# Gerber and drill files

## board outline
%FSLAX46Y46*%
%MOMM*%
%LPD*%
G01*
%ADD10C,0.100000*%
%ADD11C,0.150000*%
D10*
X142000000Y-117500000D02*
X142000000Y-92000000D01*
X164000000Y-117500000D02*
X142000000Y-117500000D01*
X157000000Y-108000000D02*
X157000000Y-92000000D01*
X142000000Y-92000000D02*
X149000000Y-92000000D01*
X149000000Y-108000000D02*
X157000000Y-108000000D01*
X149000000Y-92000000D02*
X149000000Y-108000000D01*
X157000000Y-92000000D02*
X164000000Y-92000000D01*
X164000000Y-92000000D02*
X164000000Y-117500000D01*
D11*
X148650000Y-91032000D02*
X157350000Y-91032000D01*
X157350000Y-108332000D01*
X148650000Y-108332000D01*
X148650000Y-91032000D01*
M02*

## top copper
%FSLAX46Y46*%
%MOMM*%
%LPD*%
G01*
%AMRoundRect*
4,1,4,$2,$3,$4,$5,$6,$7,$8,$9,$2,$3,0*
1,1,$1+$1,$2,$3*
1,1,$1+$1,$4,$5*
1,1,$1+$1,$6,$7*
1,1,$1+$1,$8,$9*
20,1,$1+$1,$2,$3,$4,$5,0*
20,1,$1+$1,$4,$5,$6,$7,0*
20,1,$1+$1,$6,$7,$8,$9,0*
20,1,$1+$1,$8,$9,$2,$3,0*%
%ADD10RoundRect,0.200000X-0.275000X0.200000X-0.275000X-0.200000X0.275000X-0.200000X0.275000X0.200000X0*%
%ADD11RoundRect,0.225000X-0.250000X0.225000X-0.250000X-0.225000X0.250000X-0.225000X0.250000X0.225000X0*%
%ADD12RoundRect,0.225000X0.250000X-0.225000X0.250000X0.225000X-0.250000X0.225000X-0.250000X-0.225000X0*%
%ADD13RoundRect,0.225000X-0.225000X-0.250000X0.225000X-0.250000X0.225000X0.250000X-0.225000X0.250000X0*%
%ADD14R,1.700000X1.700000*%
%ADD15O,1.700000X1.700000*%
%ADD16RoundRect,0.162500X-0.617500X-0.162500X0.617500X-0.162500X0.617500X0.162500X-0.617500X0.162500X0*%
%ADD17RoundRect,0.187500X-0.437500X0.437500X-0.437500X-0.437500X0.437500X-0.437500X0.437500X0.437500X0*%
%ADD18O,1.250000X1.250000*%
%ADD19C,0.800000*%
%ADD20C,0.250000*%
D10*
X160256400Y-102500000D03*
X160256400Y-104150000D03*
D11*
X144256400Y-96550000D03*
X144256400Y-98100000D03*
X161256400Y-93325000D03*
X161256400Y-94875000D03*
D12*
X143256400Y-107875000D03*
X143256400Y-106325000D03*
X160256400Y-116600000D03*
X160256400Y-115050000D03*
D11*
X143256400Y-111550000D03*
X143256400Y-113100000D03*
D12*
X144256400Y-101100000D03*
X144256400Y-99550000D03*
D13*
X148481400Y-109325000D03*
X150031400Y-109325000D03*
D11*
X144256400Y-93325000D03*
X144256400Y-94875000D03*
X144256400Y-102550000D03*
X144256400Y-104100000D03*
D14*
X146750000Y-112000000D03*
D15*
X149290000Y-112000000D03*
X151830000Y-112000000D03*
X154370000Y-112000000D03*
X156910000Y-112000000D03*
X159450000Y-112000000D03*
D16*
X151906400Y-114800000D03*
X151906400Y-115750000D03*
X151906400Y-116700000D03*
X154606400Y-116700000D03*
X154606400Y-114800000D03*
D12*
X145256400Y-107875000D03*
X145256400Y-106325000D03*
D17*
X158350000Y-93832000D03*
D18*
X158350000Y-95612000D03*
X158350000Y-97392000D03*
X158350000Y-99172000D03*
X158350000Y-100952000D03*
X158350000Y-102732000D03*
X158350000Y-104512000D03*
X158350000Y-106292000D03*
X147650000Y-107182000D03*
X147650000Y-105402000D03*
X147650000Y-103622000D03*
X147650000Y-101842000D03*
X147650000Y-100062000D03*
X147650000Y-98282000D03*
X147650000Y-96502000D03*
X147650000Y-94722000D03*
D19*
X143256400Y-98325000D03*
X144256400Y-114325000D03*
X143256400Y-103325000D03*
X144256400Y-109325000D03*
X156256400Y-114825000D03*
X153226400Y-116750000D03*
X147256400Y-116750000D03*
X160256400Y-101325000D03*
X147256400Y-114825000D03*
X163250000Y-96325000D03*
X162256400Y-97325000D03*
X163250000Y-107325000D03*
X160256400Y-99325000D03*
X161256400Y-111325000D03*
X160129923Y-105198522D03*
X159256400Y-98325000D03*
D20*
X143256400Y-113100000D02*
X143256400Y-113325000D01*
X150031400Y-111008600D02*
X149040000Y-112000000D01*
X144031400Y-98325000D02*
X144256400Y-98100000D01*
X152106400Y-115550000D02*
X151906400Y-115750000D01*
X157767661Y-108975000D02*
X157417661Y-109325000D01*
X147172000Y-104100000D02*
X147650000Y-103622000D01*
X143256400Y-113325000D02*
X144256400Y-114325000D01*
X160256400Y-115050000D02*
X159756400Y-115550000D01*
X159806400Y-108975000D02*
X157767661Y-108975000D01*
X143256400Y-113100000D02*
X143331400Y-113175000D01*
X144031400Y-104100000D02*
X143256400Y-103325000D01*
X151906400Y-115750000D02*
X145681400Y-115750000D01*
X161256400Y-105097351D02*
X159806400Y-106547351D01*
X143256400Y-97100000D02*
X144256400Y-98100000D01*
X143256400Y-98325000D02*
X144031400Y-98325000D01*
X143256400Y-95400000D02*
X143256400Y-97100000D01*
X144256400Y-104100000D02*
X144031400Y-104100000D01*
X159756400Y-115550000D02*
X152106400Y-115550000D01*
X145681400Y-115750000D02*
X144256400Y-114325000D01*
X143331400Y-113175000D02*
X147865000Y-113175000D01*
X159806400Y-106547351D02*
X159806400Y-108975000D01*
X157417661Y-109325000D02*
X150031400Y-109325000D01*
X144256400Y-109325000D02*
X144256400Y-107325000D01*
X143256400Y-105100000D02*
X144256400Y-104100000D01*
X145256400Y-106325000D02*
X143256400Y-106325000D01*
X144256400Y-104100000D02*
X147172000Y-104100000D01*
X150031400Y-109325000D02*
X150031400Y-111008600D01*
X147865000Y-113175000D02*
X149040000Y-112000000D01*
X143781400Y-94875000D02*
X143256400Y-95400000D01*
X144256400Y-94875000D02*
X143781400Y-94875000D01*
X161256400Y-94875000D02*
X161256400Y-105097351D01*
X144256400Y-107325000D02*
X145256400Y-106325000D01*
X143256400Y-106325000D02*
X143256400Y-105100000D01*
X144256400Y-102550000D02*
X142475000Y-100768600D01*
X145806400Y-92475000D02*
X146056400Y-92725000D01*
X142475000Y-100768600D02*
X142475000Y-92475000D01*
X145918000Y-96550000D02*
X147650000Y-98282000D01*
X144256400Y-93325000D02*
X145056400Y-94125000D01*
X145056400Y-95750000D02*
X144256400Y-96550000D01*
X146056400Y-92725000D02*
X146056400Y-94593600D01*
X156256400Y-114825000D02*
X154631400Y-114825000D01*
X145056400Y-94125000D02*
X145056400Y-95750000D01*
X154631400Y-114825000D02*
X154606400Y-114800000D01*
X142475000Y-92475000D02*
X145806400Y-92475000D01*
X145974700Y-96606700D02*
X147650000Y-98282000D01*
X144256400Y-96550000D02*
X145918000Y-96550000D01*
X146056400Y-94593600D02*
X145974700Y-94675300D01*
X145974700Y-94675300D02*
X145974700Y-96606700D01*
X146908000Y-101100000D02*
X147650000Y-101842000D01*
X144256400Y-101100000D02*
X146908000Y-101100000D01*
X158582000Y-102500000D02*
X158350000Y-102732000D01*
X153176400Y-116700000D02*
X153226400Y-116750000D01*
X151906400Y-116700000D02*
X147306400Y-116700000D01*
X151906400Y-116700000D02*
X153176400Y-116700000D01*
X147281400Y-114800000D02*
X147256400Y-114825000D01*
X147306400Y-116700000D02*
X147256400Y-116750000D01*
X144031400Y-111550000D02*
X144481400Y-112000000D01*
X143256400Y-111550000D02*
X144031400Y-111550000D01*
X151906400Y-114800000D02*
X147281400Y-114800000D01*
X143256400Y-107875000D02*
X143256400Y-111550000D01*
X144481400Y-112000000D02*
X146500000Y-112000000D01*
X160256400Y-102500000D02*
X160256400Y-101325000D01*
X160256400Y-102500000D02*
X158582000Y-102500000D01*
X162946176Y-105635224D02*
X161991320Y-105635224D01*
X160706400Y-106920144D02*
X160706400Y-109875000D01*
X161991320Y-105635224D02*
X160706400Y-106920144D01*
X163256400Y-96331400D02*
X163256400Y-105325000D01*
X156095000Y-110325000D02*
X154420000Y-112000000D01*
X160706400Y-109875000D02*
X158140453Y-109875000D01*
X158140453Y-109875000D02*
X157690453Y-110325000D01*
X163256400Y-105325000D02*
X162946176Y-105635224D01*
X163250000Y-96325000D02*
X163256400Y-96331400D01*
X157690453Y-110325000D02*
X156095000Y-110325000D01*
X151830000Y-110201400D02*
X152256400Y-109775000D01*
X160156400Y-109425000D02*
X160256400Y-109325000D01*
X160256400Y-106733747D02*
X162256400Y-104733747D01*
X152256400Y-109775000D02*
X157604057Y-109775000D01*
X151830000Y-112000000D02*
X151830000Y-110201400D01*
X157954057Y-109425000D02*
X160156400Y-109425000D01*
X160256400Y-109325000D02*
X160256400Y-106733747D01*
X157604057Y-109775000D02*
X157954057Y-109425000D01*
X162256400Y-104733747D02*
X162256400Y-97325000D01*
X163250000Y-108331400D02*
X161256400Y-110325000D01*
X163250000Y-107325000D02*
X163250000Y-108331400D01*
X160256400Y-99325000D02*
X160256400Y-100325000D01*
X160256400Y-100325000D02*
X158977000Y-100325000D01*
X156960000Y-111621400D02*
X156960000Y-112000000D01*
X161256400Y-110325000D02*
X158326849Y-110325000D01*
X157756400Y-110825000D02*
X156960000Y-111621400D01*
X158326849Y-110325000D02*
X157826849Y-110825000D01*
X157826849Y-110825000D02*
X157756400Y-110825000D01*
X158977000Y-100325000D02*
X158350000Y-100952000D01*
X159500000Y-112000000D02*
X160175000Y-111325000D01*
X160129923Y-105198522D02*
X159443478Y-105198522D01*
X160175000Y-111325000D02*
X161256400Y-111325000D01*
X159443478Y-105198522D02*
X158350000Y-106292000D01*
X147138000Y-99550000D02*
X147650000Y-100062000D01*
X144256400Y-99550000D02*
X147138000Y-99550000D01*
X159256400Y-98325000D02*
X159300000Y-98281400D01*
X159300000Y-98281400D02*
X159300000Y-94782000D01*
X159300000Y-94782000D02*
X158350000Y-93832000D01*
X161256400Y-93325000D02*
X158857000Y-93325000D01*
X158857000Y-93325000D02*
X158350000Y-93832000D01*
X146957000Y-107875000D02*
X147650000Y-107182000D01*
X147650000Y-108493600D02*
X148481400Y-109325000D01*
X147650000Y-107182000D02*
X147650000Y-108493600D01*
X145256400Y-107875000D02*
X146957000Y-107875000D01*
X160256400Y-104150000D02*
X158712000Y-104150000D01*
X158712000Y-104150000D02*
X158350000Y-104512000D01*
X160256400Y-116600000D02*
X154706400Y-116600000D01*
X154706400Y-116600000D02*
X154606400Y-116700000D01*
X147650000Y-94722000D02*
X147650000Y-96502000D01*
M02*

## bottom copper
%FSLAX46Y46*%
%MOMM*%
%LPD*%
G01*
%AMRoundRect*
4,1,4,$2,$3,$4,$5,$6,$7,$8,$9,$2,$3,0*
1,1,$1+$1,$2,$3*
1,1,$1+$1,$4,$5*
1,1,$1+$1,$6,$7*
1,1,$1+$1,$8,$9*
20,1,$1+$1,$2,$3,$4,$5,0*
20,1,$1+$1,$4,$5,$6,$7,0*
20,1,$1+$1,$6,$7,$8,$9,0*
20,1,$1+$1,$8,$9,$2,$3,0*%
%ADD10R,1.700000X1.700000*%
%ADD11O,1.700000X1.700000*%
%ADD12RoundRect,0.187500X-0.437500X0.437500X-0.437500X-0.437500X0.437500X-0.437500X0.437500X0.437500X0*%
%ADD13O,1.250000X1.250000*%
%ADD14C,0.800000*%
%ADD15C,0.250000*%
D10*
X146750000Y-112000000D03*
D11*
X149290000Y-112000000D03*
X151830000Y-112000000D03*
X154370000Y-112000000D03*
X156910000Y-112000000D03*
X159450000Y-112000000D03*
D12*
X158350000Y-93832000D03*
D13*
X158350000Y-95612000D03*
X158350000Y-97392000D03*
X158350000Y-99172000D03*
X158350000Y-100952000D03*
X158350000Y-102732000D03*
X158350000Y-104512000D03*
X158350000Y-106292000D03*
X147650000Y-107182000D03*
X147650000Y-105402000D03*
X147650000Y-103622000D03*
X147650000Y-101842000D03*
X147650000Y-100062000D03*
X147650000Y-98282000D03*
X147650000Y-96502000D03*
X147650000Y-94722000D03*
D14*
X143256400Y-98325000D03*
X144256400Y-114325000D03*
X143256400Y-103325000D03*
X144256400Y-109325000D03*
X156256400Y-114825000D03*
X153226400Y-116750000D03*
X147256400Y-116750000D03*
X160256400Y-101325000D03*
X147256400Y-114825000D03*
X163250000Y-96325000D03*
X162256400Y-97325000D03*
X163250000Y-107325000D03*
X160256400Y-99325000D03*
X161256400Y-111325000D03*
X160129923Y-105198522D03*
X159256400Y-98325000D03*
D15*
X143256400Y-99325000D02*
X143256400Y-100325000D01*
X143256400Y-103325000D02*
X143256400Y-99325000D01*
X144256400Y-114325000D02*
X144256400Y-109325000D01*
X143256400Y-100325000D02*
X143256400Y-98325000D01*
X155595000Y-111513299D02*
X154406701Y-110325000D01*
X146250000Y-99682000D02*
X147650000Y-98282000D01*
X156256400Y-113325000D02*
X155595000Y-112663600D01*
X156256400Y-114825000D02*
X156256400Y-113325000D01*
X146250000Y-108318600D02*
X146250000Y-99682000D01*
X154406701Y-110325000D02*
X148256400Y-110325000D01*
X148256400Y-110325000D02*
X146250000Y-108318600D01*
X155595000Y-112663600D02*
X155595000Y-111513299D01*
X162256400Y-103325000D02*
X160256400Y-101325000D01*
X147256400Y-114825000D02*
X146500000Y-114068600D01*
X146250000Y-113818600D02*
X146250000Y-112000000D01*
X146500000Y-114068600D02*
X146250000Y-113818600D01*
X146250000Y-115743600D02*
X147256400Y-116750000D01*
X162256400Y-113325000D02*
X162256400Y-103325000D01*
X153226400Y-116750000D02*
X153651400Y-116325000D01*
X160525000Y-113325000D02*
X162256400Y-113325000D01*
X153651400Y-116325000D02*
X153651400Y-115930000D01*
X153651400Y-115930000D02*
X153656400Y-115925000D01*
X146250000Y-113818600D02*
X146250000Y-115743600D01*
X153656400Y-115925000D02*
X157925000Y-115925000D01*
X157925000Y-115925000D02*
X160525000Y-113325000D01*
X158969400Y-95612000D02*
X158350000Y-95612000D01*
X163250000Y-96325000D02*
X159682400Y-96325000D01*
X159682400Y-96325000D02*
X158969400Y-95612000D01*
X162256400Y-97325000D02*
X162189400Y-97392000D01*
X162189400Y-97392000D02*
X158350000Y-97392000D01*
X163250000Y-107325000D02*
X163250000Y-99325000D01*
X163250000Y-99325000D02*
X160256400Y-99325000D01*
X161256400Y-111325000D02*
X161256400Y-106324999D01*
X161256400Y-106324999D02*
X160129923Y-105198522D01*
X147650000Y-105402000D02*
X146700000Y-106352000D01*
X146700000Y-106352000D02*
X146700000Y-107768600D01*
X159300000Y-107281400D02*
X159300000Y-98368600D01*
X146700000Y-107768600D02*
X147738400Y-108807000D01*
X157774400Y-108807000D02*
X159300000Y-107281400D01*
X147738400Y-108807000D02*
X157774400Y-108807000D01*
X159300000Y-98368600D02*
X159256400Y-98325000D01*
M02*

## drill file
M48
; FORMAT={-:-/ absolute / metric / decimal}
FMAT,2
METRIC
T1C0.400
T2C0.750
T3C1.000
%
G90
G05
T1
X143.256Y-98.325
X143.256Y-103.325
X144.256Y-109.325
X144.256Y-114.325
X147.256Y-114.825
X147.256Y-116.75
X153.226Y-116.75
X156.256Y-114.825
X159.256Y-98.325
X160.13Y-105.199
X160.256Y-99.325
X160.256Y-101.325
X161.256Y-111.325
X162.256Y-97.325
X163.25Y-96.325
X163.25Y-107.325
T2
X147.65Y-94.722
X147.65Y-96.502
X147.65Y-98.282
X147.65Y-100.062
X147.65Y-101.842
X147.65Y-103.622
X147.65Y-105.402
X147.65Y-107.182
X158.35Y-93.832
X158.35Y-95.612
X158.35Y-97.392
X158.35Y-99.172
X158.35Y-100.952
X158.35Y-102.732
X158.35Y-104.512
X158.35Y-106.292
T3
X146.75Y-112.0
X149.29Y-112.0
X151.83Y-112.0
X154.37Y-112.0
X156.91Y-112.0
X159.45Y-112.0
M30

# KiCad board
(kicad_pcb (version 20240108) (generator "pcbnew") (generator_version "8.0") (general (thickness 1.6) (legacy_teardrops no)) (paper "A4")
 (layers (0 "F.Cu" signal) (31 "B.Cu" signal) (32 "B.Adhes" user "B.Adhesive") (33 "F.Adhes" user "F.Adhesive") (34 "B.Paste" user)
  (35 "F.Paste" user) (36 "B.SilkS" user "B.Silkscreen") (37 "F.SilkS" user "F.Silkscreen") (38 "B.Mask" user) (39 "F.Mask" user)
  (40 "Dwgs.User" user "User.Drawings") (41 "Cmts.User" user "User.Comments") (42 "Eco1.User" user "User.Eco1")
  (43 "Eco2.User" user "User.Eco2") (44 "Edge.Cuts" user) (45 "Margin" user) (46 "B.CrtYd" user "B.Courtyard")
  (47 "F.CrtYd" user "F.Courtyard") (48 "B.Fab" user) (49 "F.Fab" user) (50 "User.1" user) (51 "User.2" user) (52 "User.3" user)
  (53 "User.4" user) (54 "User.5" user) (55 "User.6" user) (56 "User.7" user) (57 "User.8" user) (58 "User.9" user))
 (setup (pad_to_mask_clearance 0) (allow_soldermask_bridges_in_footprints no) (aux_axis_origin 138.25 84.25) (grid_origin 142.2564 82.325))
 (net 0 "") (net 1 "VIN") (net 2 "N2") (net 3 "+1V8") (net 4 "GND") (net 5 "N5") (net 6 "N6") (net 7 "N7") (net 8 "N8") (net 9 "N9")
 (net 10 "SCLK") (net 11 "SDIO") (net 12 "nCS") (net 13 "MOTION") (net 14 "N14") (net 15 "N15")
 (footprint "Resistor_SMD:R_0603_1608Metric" (layer "F.Cu") (at 160.2564 103.325 -90)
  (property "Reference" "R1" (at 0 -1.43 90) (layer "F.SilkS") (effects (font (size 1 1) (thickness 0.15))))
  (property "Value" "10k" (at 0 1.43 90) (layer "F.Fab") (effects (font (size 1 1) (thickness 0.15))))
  (pad "1" smd roundrect (at -0.825 0 270) (size 0.8 0.95) (layers "F.Cu" "F.Paste" "F.Mask") (roundrect_rratio 0.25) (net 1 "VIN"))
  (pad "2" smd roundrect (at 0.825 0 270) (size 0.8 0.95) (layers "F.Cu" "F.Paste" "F.Mask") (roundrect_rratio 0.25) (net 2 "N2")))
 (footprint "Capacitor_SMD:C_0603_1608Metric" (layer "F.Cu") (at 144.2564 97.325 -90)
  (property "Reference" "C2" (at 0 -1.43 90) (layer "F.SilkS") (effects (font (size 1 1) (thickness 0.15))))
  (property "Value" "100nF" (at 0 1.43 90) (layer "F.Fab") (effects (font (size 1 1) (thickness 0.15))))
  (pad "1" smd roundrect (at -0.775 0 270) (size 0.9 0.95) (layers "F.Cu" "F.Paste" "F.Mask") (roundrect_rratio 0.25) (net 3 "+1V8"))
  (pad "2" smd roundrect (at 0.775 0 270) (size 0.9 0.95) (layers "F.Cu" "F.Paste" "F.Mask") (roundrect_rratio 0.25) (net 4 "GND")))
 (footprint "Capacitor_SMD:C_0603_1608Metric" (layer "F.Cu") (at 161.2564 94.1 -90)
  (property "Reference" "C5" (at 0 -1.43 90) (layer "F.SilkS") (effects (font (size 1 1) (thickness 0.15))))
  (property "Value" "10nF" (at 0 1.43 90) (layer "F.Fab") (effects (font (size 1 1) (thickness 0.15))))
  (pad "1" smd roundrect (at -0.775 0 270) (size 0.9 0.95) (layers "F.Cu" "F.Paste" "F.Mask") (roundrect_rratio 0.25) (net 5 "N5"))
  (pad "2" smd roundrect (at 0.775 0 270) (size 0.9 0.95) (layers "F.Cu" "F.Paste" "F.Mask") (roundrect_rratio 0.25) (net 4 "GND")))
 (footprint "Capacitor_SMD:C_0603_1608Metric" (layer "F.Cu") (at 143.2564 107.1 90)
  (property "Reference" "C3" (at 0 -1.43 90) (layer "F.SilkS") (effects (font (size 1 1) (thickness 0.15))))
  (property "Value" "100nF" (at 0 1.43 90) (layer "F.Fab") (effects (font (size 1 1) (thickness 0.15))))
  (pad "1" smd roundrect (at -0.775 0 90) (size 0.9 0.95) (layers "F.Cu" "F.Paste" "F.Mask") (roundrect_rratio 0.25) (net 1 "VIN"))
  (pad "2" smd roundrect (at 0.775 0 90) (size 0.9 0.95) (layers "F.Cu" "F.Paste" "F.Mask") (roundrect_rratio 0.25) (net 4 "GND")))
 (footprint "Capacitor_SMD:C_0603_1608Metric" (layer "F.Cu") (at 160.2564 115.825 90)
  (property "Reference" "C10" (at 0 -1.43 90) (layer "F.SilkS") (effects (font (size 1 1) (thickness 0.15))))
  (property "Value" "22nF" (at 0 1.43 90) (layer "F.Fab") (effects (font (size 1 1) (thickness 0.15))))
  (pad "1" smd roundrect (at -0.775 0 90) (size 0.9 0.95) (layers "F.Cu" "F.Paste" "F.Mask") (roundrect_rratio 0.25) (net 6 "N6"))
  (pad "2" smd roundrect (at 0.775 0 90) (size 0.9 0.95) (layers "F.Cu" "F.Paste" "F.Mask") (roundrect_rratio 0.25) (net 4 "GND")))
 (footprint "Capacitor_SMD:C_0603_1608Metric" (layer "F.Cu") (at 143.2564 112.325 -90)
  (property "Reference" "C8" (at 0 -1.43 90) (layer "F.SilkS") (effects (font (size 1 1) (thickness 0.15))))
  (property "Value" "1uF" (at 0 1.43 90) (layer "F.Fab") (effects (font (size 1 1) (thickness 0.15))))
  (pad "1" smd roundrect (at -0.775 0 270) (size 0.9 0.95) (layers "F.Cu" "F.Paste" "F.Mask") (roundrect_rratio 0.25) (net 1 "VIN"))
  (pad "2" smd roundrect (at 0.775 0 270) (size 0.9 0.95) (layers "F.Cu" "F.Paste" "F.Mask") (roundrect_rratio 0.25) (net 4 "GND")))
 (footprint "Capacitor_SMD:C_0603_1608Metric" (layer "F.Cu") (at 144.2564 100.325 90)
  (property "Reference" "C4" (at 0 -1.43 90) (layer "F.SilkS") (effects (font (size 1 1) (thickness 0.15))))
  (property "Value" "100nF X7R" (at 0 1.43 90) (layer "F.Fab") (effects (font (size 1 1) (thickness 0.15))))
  (pad "1" smd roundrect (at -0.775 0 90) (size 0.9 0.95) (layers "F.Cu" "F.Paste" "F.Mask") (roundrect_rratio 0.25) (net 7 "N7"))
  (pad "2" smd roundrect (at 0.775 0 90) (size 0.9 0.95) (layers "F.Cu" "F.Paste" "F.Mask") (roundrect_rratio 0.25) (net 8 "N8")))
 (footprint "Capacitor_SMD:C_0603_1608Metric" (layer "F.Cu") (at 149.2564 109.325)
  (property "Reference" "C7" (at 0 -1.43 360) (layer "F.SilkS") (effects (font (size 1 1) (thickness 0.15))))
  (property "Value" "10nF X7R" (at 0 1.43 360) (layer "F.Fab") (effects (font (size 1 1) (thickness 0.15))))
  (pad "1" smd roundrect (at -0.775 0) (size 0.9 0.95) (layers "F.Cu" "F.Paste" "F.Mask") (roundrect_rratio 0.25) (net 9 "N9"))
  (pad "2" smd roundrect (at 0.775 0) (size 0.9 0.95) (layers "F.Cu" "F.Paste" "F.Mask") (roundrect_rratio 0.25) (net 4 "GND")))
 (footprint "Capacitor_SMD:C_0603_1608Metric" (layer "F.Cu") (at 144.2564 94.1 -90)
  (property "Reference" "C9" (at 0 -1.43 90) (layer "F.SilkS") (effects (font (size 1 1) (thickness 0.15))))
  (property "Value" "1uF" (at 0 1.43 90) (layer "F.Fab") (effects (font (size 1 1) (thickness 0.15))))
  (pad "1" smd roundrect (at -0.775 0 270) (size 0.9 0.95) (layers "F.Cu" "F.Paste" "F.Mask") (roundrect_rratio 0.25) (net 3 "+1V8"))
  (pad "2" smd roundrect (at 0.775 0 270) (size 0.9 0.95) (layers "F.Cu" "F.Paste" "F.Mask") (roundrect_rratio 0.25) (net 4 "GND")))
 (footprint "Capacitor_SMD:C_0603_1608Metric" (layer "F.Cu") (at 144.2564 103.325 -90)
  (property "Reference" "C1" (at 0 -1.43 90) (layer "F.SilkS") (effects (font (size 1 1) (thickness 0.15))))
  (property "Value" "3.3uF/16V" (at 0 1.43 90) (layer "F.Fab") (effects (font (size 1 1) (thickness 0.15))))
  (pad "1" smd roundrect (at -0.775 0 270) (size 0.9 0.95) (layers "F.Cu" "F.Paste" "F.Mask") (roundrect_rratio 0.25) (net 3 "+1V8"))
  (pad "2" smd roundrect (at 0.775 0 270) (size 0.9 0.95) (layers "F.Cu" "F.Paste" "F.Mask") (roundrect_rratio 0.25) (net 4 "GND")))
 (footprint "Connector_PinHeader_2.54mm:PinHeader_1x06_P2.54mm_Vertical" (layer "F.Cu") (at 146.75 112 90)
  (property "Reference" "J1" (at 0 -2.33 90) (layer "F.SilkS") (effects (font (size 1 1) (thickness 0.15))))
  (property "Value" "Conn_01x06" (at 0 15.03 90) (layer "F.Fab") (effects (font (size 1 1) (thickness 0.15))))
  (pad "1" thru_hole rect (at 0 0 90) (size 1.7 1.7) (drill 1) (layers "*.Cu" "*.Mask") (remove_unused_layers no) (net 1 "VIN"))
  (pad "2" thru_hole oval (at 0 2.54 90) (size 1.7 1.7) (drill 1) (layers "*.Cu" "*.Mask") (remove_unused_layers no) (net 4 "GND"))
  (pad "3" thru_hole oval (at 0 5.08 90) (size 1.7 1.7) (drill 1) (layers "*.Cu" "*.Mask") (remove_unused_layers no) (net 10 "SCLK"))
  (pad "4" thru_hole oval (at 0 7.62 90) (size 1.7 1.7) (drill 1) (layers "*.Cu" "*.Mask") (remove_unused_layers no) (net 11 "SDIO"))
  (pad "5" thru_hole oval (at 0 10.16 90) (size 1.7 1.7) (drill 1) (layers "*.Cu" "*.Mask") (remove_unused_layers no) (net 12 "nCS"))
  (pad "6" thru_hole oval (at 0 12.7 90) (size 1.7 1.7) (drill 1) (layers "*.Cu" "*.Mask") (remove_unused_layers no) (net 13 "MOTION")))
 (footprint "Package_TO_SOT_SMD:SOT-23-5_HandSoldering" (layer "F.Cu") (at 153.2564 115.75)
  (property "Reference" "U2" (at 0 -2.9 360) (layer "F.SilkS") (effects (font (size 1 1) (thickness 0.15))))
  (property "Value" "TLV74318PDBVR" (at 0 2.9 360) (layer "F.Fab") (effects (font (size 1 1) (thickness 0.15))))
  (pad "1" smd roundrect (at -1.35 -0.95) (size 1.56 0.65) (layers "F.Cu" "F.Paste" "F.Mask") (roundrect_rratio 0.25) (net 1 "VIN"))
  (pad "2" smd roundrect (at -1.35 0) (size 1.56 0.65) (layers "F.Cu" "F.Paste" "F.Mask") (roundrect_rratio 0.25) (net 4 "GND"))
  (pad "3" smd roundrect (at -1.35 0.95) (size 1.56 0.65) (layers "F.Cu" "F.Paste" "F.Mask") (roundrect_rratio 0.25) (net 1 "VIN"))
  (pad "4" smd roundrect (at 1.35 0.95) (size 1.56 0.65) (layers "F.Cu" "F.Paste" "F.Mask") (roundrect_rratio 0.25) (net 6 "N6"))
  (pad "5" smd roundrect (at 1.35 -0.95) (size 1.56 0.65) (layers "F.Cu" "F.Paste" "F.Mask") (roundrect_rratio 0.25) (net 3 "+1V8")))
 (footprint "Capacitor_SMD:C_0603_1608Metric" (layer "F.Cu") (at 145.2564 107.1 90)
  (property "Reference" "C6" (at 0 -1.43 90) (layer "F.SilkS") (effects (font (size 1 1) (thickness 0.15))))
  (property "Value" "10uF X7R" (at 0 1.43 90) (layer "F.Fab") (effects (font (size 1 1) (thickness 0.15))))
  (pad "1" smd roundrect (at -0.775 0 90) (size 0.9 0.95) (layers "F.Cu" "F.Paste" "F.Mask") (roundrect_rratio 0.25) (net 9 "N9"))
  (pad "2" smd roundrect (at 0.775 0 90) (size 0.9 0.95) (layers "F.Cu" "F.Paste" "F.Mask") (roundrect_rratio 0.25) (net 4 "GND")))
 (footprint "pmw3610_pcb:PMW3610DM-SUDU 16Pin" (layer "B.Cu") (at 153 100 90)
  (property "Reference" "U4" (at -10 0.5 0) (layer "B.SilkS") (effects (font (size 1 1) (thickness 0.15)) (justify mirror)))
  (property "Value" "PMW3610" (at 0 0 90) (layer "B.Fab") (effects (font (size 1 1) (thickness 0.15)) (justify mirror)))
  (fp_rect (start -8.332 -4.35) (end 8.968 4.35) (stroke (width 0.15) (type solid)) (fill none) (layer "Edge.Cuts"))
  (pad "1" thru_hole roundrect (at 6.168 5.35 270) (size 1.25 1.25) (drill 0.75) (layers "*.Cu" "*.Mask") (remove_unused_layers no)
   (roundrect_rratio 0.15) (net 5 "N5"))
  (pad "2" thru_hole oval (at 4.388 5.35 270) (size 1.25 1.25) (drill 0.75) (layers "*.Cu" "*.Mask") (remove_unused_layers no)
   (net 11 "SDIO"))
  (pad "3" thru_hole oval (at 2.608 5.35 270) (size 1.25 1.25) (drill 0.75) (layers "*.Cu" "*.Mask") (remove_unused_layers no)
   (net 10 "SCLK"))
  (pad "4" thru_hole oval (at 0.828 5.35 270) (size 1.25 1.25) (drill 0.75) (layers "*.Cu" "*.Mask") (remove_unused_layers no)
   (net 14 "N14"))
  (pad "5" thru_hole oval (at -0.952 5.35 270) (size 1.25 1.25) (drill 0.75) (layers "*.Cu" "*.Mask") (remove_unused_layers no)
   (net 12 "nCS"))
  (pad "6" thru_hole oval (at -2.732 5.35 270) (size 1.25 1.25) (drill 0.75) (layers "*.Cu" "*.Mask") (remove_unused_layers no)
   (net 1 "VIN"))
  (pad "7" thru_hole oval (at -4.512 5.35 270) (size 1.25 1.25) (drill 0.75) (layers "*.Cu" "*.Mask") (remove_unused_layers no) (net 2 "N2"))
  (pad "8" thru_hole oval (at -6.292 5.35 270) (size 1.25 1.25) (drill 0.75) (layers "*.Cu" "*.Mask") (remove_unused_layers no)
   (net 13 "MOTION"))
  (pad "9" thru_hole oval (at -7.182 -5.35 270) (size 1.25 1.25) (drill 0.75) (layers "*.Cu" "*.Mask") (remove_unused_layers no)
   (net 9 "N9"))
  (pad "10" thru_hole oval (at -5.402 -5.35 270) (size 1.25 1.25) (drill 0.75) (layers "*.Cu" "*.Mask") (remove_unused_layers no)
   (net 5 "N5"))
  (pad "11" thru_hole oval (at -3.622 -5.35 270) (size 1.25 1.25) (drill 0.75) (layers "*.Cu" "*.Mask") (remove_unused_layers no)
   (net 4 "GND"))
  (pad "12" thru_hole oval (at -1.842 -5.35 270) (size 1.25 1.25) (drill 0.75) (layers "*.Cu" "*.Mask") (remove_unused_layers no)
   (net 7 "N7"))
  (pad "13" thru_hole oval (at -0.062 -5.35 270) (size 1.25 1.25) (drill 0.75) (layers "*.Cu" "*.Mask") (remove_unused_layers no)
   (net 8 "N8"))
  (pad "14" thru_hole oval (at 1.718 -5.35 270) (size 1.25 1.25) (drill 0.75) (layers "*.Cu" "*.Mask") (remove_unused_layers no)
   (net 3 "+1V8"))
  (pad "15" thru_hole oval (at 3.498 -5.35 270) (size 1.25 1.25) (drill 0.75) (layers "*.Cu" "*.Mask") (remove_unused_layers no)
   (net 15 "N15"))
  (pad "16" thru_hole oval (at 5.278 -5.35 270) (size 1.25 1.25) (drill 0.75) (layers "*.Cu" "*.Mask") (remove_unused_layers no)
   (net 15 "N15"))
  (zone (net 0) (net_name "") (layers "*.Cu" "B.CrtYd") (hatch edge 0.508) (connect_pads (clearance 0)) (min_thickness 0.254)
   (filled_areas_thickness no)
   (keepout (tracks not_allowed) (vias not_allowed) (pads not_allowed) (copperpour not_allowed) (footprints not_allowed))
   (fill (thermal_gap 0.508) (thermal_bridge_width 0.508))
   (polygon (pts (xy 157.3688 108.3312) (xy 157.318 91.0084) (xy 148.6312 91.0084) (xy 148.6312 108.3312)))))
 (gr_line (start 142 117.5) (end 142 92) (stroke (width 0.1) (type default)) (layer "Edge.Cuts"))
 (gr_line (start 164 117.5) (end 142 117.5) (stroke (width 0.1) (type default)) (layer "Edge.Cuts"))
 (gr_line (start 157 108) (end 157 92) (stroke (width 0.1) (type default)) (layer "Edge.Cuts"))
 (gr_line (start 142 92) (end 149 92) (stroke (width 0.1) (type default)) (layer "Edge.Cuts"))
 (gr_line (start 149 108) (end 157 108) (stroke (width 0.1) (type default)) (layer "Edge.Cuts"))
 (gr_line (start 149 92) (end 149 108) (stroke (width 0.1) (type default)) (layer "Edge.Cuts"))
 (gr_line (start 157 92) (end 164 92) (stroke (width 0.1) (type default)) (layer "Edge.Cuts"))
 (gr_line (start 164 92) (end 164 117.5) (stroke (width 0.1) (type default)) (layer "Edge.Cuts"))
 (segment (start 143.2564 113.1) (end 143.2564 113.325) (width 0.25) (layer "F.Cu") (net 4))
 (segment (start 150.0314 111.0086) (end 149.04 112) (width 0.25) (layer "F.Cu") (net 4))
 (segment (start 144.0314 98.325) (end 144.2564 98.1) (width 0.25) (layer "F.Cu") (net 4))
 (segment (start 152.1064 115.55) (end 151.9064 115.75) (width 0.25) (layer "F.Cu") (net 4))
 (segment (start 157.767661 108.975) (end 157.417661 109.325) (width 0.25) (layer "F.Cu") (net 4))
 (segment (start 147.172 104.1) (end 147.65 103.622) (width 0.25) (layer "F.Cu") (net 4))
 (segment (start 143.2564 113.325) (end 144.2564 114.325) (width 0.25) (layer "F.Cu") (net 4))
 (segment (start 160.2564 115.05) (end 159.7564 115.55) (width 0.25) (layer "F.Cu") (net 4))
 (segment (start 159.8064 108.975) (end 157.767661 108.975) (width 0.25) (layer "F.Cu") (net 4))
 (segment (start 143.2564 113.1) (end 143.3314 113.175) (width 0.25) (layer "F.Cu") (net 4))
 (segment (start 144.0314 104.1) (end 143.2564 103.325) (width 0.25) (layer "F.Cu") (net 4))
 (segment (start 151.9064 115.75) (end 145.6814 115.75) (width 0.25) (layer "F.Cu") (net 4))
 (segment (start 161.2564 105.097351) (end 159.8064 106.547351) (width 0.25) (layer "F.Cu") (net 4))
 (segment (start 143.2564 97.1) (end 144.2564 98.1) (width 0.25) (layer "F.Cu") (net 4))
 (segment (start 143.2564 98.325) (end 144.0314 98.325) (width 0.25) (layer "F.Cu") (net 4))
 (segment (start 143.2564 95.4) (end 143.2564 97.1) (width 0.25) (layer "F.Cu") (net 4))
 (segment (start 144.2564 104.1) (end 144.0314 104.1) (width 0.25) (layer "F.Cu") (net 4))
 (segment (start 159.7564 115.55) (end 152.1064 115.55) (width 0.25) (layer "F.Cu") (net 4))
 (segment (start 145.6814 115.75) (end 144.2564 114.325) (width 0.25) (layer "F.Cu") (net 4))
 (segment (start 143.3314 113.175) (end 147.865 113.175) (width 0.25) (layer "F.Cu") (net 4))
 (segment (start 159.8064 106.547351) (end 159.8064 108.975) (width 0.25) (layer "F.Cu") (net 4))
 (segment (start 157.417661 109.325) (end 150.0314 109.325) (width 0.25) (layer "F.Cu") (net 4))
 (segment (start 144.2564 109.325) (end 144.2564 107.325) (width 0.25) (layer "F.Cu") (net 4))
 (segment (start 143.2564 105.1) (end 144.2564 104.1) (width 0.25) (layer "F.Cu") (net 4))
 (segment (start 145.2564 106.325) (end 143.2564 106.325) (width 0.25) (layer "F.Cu") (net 4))
 (segment (start 144.2564 104.1) (end 147.172 104.1) (width 0.25) (layer "F.Cu") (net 4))
 (segment (start 150.0314 109.325) (end 150.0314 111.0086) (width 0.25) (layer "F.Cu") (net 4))
 (segment (start 147.865 113.175) (end 149.04 112) (width 0.25) (layer "F.Cu") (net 4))
 (segment (start 143.7814 94.875) (end 143.2564 95.4) (width 0.25) (layer "F.Cu") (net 4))
 (segment (start 144.2564 94.875) (end 143.7814 94.875) (width 0.25) (layer "F.Cu") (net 4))
 (segment (start 161.2564 94.875) (end 161.2564 105.097351) (width 0.25) (layer "F.Cu") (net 4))
 (segment (start 144.2564 107.325) (end 145.2564 106.325) (width 0.25) (layer "F.Cu") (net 4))
 (segment (start 143.2564 106.325) (end 143.2564 105.1) (width 0.25) (layer "F.Cu") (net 4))
 (via (at 143.2564 98.325) (size 0.8) (drill 0.4) (layers "F.Cu" "B.Cu") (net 4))
 (via (at 144.2564 114.325) (size 0.8) (drill 0.4) (layers "F.Cu" "B.Cu") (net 4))
 (via (at 143.2564 103.325) (size 0.8) (drill 0.4) (layers "F.Cu" "B.Cu") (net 4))
 (via (at 144.2564 109.325) (size 0.8) (drill 0.4) (layers "F.Cu" "B.Cu") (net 4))
 (segment (start 143.2564 99.325) (end 143.2564 100.325) (width 0.25) (layer "B.Cu") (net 4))
 (segment (start 143.2564 103.325) (end 143.2564 99.325) (width 0.25) (layer "B.Cu") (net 4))
 (segment (start 144.2564 114.325) (end 144.2564 109.325) (width 0.25) (layer "B.Cu") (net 4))
 (segment (start 143.2564 100.325) (end 143.2564 98.325) (width 0.25) (layer "B.Cu") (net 4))
 (segment (start 144.2564 102.55) (end 142.475 100.7686) (width 0.25) (layer "F.Cu") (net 3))
 (segment (start 145.8064 92.475) (end 146.0564 92.725) (width 0.25) (layer "F.Cu") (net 3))
 (segment (start 142.475 100.7686) (end 142.475 92.475) (width 0.25) (layer "F.Cu") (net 3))
 (segment (start 145.918 96.55) (end 147.65 98.282) (width 0.25) (layer "F.Cu") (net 3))
 (segment (start 144.2564 93.325) (end 145.0564 94.125) (width 0.25) (layer "F.Cu") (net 3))
 (segment (start 145.0564 95.75) (end 144.2564 96.55) (width 0.25) (layer "F.Cu") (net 3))
 (segment (start 146.0564 92.725) (end 146.0564 94.5936) (width 0.25) (layer "F.Cu") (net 3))
 (segment (start 156.2564 114.825) (end 154.6314 114.825) (width 0.25) (layer "F.Cu") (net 3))
 (segment (start 145.0564 94.125) (end 145.0564 95.75) (width 0.25) (layer "F.Cu") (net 3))
 (segment (start 154.6314 114.825) (end 154.6064 114.8) (width 0.25) (layer "F.Cu") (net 3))
 (segment (start 142.475 92.475) (end 145.8064 92.475) (width 0.25) (layer "F.Cu") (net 3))
 (segment (start 145.9747 96.6067) (end 147.65 98.282) (width 0.25) (layer "F.Cu") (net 3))
 (segment (start 144.2564 96.55) (end 145.918 96.55) (width 0.25) (layer "F.Cu") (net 3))
 (segment (start 146.0564 94.5936) (end 145.9747 94.6753) (width 0.25) (layer "F.Cu") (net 3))
 (segment (start 145.9747 94.6753) (end 145.9747 96.6067) (width 0.25) (layer "F.Cu") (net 3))
 (via (at 156.2564 114.825) (size 0.8) (drill 0.4) (layers "F.Cu" "B.Cu") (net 3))
 (segment (start 155.595 111.513299) (end 154.406701 110.325) (width 0.25) (layer "B.Cu") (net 3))
 (segment (start 146.25 99.682) (end 147.65 98.282) (width 0.25) (layer "B.Cu") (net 3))
 (segment (start 156.2564 113.325) (end 155.595 112.6636) (width 0.25) (layer "B.Cu") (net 3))
 (segment (start 156.2564 114.825) (end 156.2564 113.325) (width 0.25) (layer "B.Cu") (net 3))
 (segment (start 146.25 108.3186) (end 146.25 99.682) (width 0.25) (layer "B.Cu") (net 3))
 (segment (start 154.406701 110.325) (end 148.2564 110.325) (width 0.25) (layer "B.Cu") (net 3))
 (segment (start 148.2564 110.325) (end 146.25 108.3186) (width 0.25) (layer "B.Cu") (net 3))
 (segment (start 155.595 112.6636) (end 155.595 111.513299) (width 0.25) (layer "B.Cu") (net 3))
 (segment (start 146.908 101.1) (end 147.65 101.842) (width 0.25) (layer "F.Cu") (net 7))
 (segment (start 144.2564 101.1) (end 146.908 101.1) (width 0.25) (layer "F.Cu") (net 7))
 (segment (start 158.582 102.5) (end 158.35 102.732) (width 0.25) (layer "F.Cu") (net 1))
 (segment (start 153.1764 116.7) (end 153.2264 116.75) (width 0.25) (layer "F.Cu") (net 1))
 (segment (start 151.9064 116.7) (end 147.3064 116.7) (width 0.25) (layer "F.Cu") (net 1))
 (segment (start 151.9064 116.7) (end 153.1764 116.7) (width 0.25) (layer "F.Cu") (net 1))
 (segment (start 147.2814 114.8) (end 147.2564 114.825) (width 0.25) (layer "F.Cu") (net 1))
 (segment (start 147.3064 116.7) (end 147.2564 116.75) (width 0.25) (layer "F.Cu") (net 1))
 (segment (start 144.0314 111.55) (end 144.4814 112) (width 0.25) (layer "F.Cu") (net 1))
 (segment (start 143.2564 111.55) (end 144.0314 111.55) (width 0.25) (layer "F.Cu") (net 1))
 (segment (start 151.9064 114.8) (end 147.2814 114.8) (width 0.25) (layer "F.Cu") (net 1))
 (segment (start 143.2564 107.875) (end 143.2564 111.55) (width 0.25) (layer "F.Cu") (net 1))
 (segment (start 144.4814 112) (end 146.5 112) (width 0.25) (layer "F.Cu") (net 1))
 (segment (start 160.2564 102.5) (end 160.2564 101.325) (width 0.25) (layer "F.Cu") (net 1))
 (segment (start 160.2564 102.5) (end 158.582 102.5) (width 0.25) (layer "F.Cu") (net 1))
 (via (at 153.2264 116.75) (size 0.8) (drill 0.4) (layers "F.Cu" "B.Cu") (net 1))
 (via (at 147.2564 116.75) (size 0.8) (drill 0.4) (layers "F.Cu" "B.Cu") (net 1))
 (via (at 160.2564 101.325) (size 0.8) (drill 0.4) (layers "F.Cu" "B.Cu") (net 1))
 (via (at 147.2564 114.825) (size 0.8) (drill 0.4) (layers "F.Cu" "B.Cu") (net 1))
 (segment (start 162.2564 103.325) (end 160.2564 101.325) (width 0.25) (layer "B.Cu") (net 1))
 (segment (start 147.2564 114.825) (end 146.5 114.0686) (width 0.25) (layer "B.Cu") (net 1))
 (segment (start 146.25 113.8186) (end 146.25 112) (width 0.25) (layer "B.Cu") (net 1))
 (segment (start 146.5 114.0686) (end 146.25 113.8186) (width 0.25) (layer "B.Cu") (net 1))
 (segment (start 146.25 115.7436) (end 147.2564 116.75) (width 0.25) (layer "B.Cu") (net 1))
 (segment (start 162.2564 113.325) (end 162.2564 103.325) (width 0.25) (layer "B.Cu") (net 1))
 (segment (start 153.2264 116.75) (end 153.6514 116.325) (width 0.25) (layer "B.Cu") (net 1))
 (segment (start 160.525 113.325) (end 162.2564 113.325) (width 0.25) (layer "B.Cu") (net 1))
 (segment (start 153.6514 116.325) (end 153.6514 115.93) (width 0.25) (layer "B.Cu") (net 1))
 (segment (start 153.6514 115.93) (end 153.6564 115.925) (width 0.25) (layer "B.Cu") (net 1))
 (segment (start 146.25 113.8186) (end 146.25 115.7436) (width 0.25) (layer "B.Cu") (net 1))
 (segment (start 153.6564 115.925) (end 157.925 115.925) (width 0.25) (layer "B.Cu") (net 1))
 (segment (start 157.925 115.925) (end 160.525 113.325) (width 0.25) (layer "B.Cu") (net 1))
 (segment (start 162.946176 105.635224) (end 161.99132 105.635224) (width 0.25) (layer "F.Cu") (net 11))
 (segment (start 160.7064 106.920144) (end 160.7064 109.875) (width 0.25) (layer "F.Cu") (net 11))
 (segment (start 161.99132 105.635224) (end 160.7064 106.920144) (width 0.25) (layer "F.Cu") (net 11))
 (segment (start 163.2564 96.3314) (end 163.2564 105.325) (width 0.25) (layer "F.Cu") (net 11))
 (segment (start 156.095 110.325) (end 154.42 112) (width 0.25) (layer "F.Cu") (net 11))
 (segment (start 160.7064 109.875) (end 158.140453 109.875) (width 0.25) (layer "F.Cu") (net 11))
 (segment (start 158.140453 109.875) (end 157.690453 110.325) (width 0.25) (layer "F.Cu") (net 11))
 (segment (start 163.2564 105.325) (end 162.946176 105.635224) (width 0.25) (layer "F.Cu") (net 11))
 (segment (start 163.25 96.325) (end 163.2564 96.3314) (width 0.25) (layer "F.Cu") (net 11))
 (segment (start 157.690453 110.325) (end 156.095 110.325) (width 0.25) (layer "F.Cu") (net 11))
 (via (at 163.25 96.325) (size 0.8) (drill 0.4) (layers "F.Cu" "B.Cu") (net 11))
 (segment (start 158.9694 95.612) (end 158.35 95.612) (width 0.25) (layer "B.Cu") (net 11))
 (segment (start 163.25 96.325) (end 159.6824 96.325) (width 0.25) (layer "B.Cu") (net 11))
 (segment (start 159.6824 96.325) (end 158.9694 95.612) (width 0.25) (layer "B.Cu") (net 11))
 (segment (start 151.83 110.2014) (end 152.2564 109.775) (width 0.25) (layer "F.Cu") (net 10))
 (segment (start 160.1564 109.425) (end 160.2564 109.325) (width 0.25) (layer "F.Cu") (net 10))
 (segment (start 160.2564 106.733747) (end 162.2564 104.733747) (width 0.25) (layer "F.Cu") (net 10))
 (segment (start 152.2564 109.775) (end 157.604057 109.775) (width 0.25) (layer "F.Cu") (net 10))
 (segment (start 151.83 112) (end 151.83 110.2014) (width 0.25) (layer "F.Cu") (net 10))
 (segment (start 157.954057 109.425) (end 160.1564 109.425) (width 0.25) (layer "F.Cu") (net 10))
 (segment (start 160.2564 109.325) (end 160.2564 106.733747) (width 0.25) (layer "F.Cu") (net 10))
 (segment (start 157.604057 109.775) (end 157.954057 109.425) (width 0.25) (layer "F.Cu") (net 10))
 (segment (start 162.2564 104.733747) (end 162.2564 97.325) (width 0.25) (layer "F.Cu") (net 10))
 (via (at 162.2564 97.325) (size 0.8) (drill 0.4) (layers "F.Cu" "B.Cu") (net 10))
 (segment (start 162.2564 97.325) (end 162.1894 97.392) (width 0.25) (layer "B.Cu") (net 10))
 (segment (start 162.1894 97.392) (end 158.35 97.392) (width 0.25) (layer "B.Cu") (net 10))
 (segment (start 163.25 108.3314) (end 161.2564 110.325) (width 0.25) (layer "F.Cu") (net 12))
 (segment (start 163.25 107.325) (end 163.25 108.3314) (width 0.25) (layer "F.Cu") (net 12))
 (segment (start 160.2564 99.325) (end 160.2564 100.325) (width 0.25) (layer "F.Cu") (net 12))
 (segment (start 160.2564 100.325) (end 158.977 100.325) (width 0.25) (layer "F.Cu") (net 12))
 (segment (start 156.96 111.6214) (end 156.96 112) (width 0.25) (layer "F.Cu") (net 12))
 (segment (start 161.2564 110.325) (end 158.326849 110.325) (width 0.25) (layer "F.Cu") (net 12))
 (segment (start 157.7564 110.825) (end 156.96 111.6214) (width 0.25) (layer "F.Cu") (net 12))
 (segment (start 158.326849 110.325) (end 157.826849 110.825) (width 0.25) (layer "F.Cu") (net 12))
 (segment (start 157.826849 110.825) (end 157.7564 110.825) (width 0.25) (layer "F.Cu") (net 12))
 (segment (start 158.977 100.325) (end 158.35 100.952) (width 0.25) (layer "F.Cu") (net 12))
 (via (at 163.25 107.325) (size 0.8) (drill 0.4) (layers "F.Cu" "B.Cu") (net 12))
 (via (at 160.2564 99.325) (size 0.8) (drill 0.4) (layers "F.Cu" "B.Cu") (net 12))
 (segment (start 163.25 107.325) (end 163.25 99.325) (width 0.25) (layer "B.Cu") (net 12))
 (segment (start 163.25 99.325) (end 160.2564 99.325) (width 0.25) (layer "B.Cu") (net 12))
 (segment (start 159.5 112) (end 160.175 111.325) (width 0.25) (layer "F.Cu") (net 13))
 (segment (start 160.129923 105.198522) (end 159.443478 105.198522) (width 0.25) (layer "F.Cu") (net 13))
 (segment (start 160.175 111.325) (end 161.2564 111.325) (width 0.25) (layer "F.Cu") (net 13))
 (segment (start 159.443478 105.198522) (end 158.35 106.292) (width 0.25) (layer "F.Cu") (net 13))
 (via (at 161.2564 111.325) (size 0.8) (drill 0.4) (layers "F.Cu" "B.Cu") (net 13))
 (via (at 160.129923 105.198522) (size 0.8) (drill 0.4) (layers "F.Cu" "B.Cu") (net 13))
 (segment (start 161.2564 111.325) (end 161.2564 106.324999) (width 0.25) (layer "B.Cu") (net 13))
 (segment (start 161.2564 106.324999) (end 160.129923 105.198522) (width 0.25) (layer "B.Cu") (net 13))
 (segment (start 147.138 99.55) (end 147.65 100.062) (width 0.25) (layer "F.Cu") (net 8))
 (segment (start 144.2564 99.55) (end 147.138 99.55) (width 0.25) (layer "F.Cu") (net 8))
 (segment (start 159.2564 98.325) (end 159.3 98.2814) (width 0.25) (layer "F.Cu") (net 5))
 (segment (start 159.3 98.2814) (end 159.3 94.782) (width 0.25) (layer "F.Cu") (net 5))
 (segment (start 159.3 94.782) (end 158.35 93.832) (width 0.25) (layer "F.Cu") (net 5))
 (segment (start 161.2564 93.325) (end 158.857 93.325) (width 0.25) (layer "F.Cu") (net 5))
 (segment (start 158.857 93.325) (end 158.35 93.832) (width 0.25) (layer "F.Cu") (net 5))
 (via (at 159.2564 98.325) (size 0.8) (drill 0.4) (layers "F.Cu" "B.Cu") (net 5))
 (segment (start 147.65 105.402) (end 146.7 106.352) (width 0.25) (layer "B.Cu") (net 5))
 (segment (start 146.7 106.352) (end 146.7 107.7686) (width 0.25) (layer "B.Cu") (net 5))
 (segment (start 159.3 107.2814) (end 159.3 98.3686) (width 0.25) (layer "B.Cu") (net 5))
 (segment (start 146.7 107.7686) (end 147.7384 108.807) (width 0.25) (layer "B.Cu") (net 5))
 (segment (start 157.7744 108.807) (end 159.3 107.2814) (width 0.25) (layer "B.Cu") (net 5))
 (segment (start 147.7384 108.807) (end 157.7744 108.807) (width 0.25) (layer "B.Cu") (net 5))
 (segment (start 159.3 98.3686) (end 159.2564 98.325) (width 0.25) (layer "B.Cu") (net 5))
 (segment (start 146.957 107.875) (end 147.65 107.182) (width 0.25) (layer "F.Cu") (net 9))
 (segment (start 147.65 108.4936) (end 148.4814 109.325) (width 0.25) (layer "F.Cu") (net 9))
 (segment (start 147.65 107.182) (end 147.65 108.4936) (width 0.25) (layer "F.Cu") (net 9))
 (segment (start 145.2564 107.875) (end 146.957 107.875) (width 0.25) (layer "F.Cu") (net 9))
 (segment (start 160.2564 104.15) (end 158.712 104.15) (width 0.25) (layer "F.Cu") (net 2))
 (segment (start 158.712 104.15) (end 158.35 104.512) (width 0.25) (layer "F.Cu") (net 2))
 (segment (start 160.2564 116.6) (end 154.7064 116.6) (width 0.25) (layer "F.Cu") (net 6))
 (segment (start 154.7064 116.6) (end 154.6064 116.7) (width 0.25) (layer "F.Cu") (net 6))
 (segment (start 147.65 94.722) (end 147.65 96.502) (width 0.25) (layer "F.Cu") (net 15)))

